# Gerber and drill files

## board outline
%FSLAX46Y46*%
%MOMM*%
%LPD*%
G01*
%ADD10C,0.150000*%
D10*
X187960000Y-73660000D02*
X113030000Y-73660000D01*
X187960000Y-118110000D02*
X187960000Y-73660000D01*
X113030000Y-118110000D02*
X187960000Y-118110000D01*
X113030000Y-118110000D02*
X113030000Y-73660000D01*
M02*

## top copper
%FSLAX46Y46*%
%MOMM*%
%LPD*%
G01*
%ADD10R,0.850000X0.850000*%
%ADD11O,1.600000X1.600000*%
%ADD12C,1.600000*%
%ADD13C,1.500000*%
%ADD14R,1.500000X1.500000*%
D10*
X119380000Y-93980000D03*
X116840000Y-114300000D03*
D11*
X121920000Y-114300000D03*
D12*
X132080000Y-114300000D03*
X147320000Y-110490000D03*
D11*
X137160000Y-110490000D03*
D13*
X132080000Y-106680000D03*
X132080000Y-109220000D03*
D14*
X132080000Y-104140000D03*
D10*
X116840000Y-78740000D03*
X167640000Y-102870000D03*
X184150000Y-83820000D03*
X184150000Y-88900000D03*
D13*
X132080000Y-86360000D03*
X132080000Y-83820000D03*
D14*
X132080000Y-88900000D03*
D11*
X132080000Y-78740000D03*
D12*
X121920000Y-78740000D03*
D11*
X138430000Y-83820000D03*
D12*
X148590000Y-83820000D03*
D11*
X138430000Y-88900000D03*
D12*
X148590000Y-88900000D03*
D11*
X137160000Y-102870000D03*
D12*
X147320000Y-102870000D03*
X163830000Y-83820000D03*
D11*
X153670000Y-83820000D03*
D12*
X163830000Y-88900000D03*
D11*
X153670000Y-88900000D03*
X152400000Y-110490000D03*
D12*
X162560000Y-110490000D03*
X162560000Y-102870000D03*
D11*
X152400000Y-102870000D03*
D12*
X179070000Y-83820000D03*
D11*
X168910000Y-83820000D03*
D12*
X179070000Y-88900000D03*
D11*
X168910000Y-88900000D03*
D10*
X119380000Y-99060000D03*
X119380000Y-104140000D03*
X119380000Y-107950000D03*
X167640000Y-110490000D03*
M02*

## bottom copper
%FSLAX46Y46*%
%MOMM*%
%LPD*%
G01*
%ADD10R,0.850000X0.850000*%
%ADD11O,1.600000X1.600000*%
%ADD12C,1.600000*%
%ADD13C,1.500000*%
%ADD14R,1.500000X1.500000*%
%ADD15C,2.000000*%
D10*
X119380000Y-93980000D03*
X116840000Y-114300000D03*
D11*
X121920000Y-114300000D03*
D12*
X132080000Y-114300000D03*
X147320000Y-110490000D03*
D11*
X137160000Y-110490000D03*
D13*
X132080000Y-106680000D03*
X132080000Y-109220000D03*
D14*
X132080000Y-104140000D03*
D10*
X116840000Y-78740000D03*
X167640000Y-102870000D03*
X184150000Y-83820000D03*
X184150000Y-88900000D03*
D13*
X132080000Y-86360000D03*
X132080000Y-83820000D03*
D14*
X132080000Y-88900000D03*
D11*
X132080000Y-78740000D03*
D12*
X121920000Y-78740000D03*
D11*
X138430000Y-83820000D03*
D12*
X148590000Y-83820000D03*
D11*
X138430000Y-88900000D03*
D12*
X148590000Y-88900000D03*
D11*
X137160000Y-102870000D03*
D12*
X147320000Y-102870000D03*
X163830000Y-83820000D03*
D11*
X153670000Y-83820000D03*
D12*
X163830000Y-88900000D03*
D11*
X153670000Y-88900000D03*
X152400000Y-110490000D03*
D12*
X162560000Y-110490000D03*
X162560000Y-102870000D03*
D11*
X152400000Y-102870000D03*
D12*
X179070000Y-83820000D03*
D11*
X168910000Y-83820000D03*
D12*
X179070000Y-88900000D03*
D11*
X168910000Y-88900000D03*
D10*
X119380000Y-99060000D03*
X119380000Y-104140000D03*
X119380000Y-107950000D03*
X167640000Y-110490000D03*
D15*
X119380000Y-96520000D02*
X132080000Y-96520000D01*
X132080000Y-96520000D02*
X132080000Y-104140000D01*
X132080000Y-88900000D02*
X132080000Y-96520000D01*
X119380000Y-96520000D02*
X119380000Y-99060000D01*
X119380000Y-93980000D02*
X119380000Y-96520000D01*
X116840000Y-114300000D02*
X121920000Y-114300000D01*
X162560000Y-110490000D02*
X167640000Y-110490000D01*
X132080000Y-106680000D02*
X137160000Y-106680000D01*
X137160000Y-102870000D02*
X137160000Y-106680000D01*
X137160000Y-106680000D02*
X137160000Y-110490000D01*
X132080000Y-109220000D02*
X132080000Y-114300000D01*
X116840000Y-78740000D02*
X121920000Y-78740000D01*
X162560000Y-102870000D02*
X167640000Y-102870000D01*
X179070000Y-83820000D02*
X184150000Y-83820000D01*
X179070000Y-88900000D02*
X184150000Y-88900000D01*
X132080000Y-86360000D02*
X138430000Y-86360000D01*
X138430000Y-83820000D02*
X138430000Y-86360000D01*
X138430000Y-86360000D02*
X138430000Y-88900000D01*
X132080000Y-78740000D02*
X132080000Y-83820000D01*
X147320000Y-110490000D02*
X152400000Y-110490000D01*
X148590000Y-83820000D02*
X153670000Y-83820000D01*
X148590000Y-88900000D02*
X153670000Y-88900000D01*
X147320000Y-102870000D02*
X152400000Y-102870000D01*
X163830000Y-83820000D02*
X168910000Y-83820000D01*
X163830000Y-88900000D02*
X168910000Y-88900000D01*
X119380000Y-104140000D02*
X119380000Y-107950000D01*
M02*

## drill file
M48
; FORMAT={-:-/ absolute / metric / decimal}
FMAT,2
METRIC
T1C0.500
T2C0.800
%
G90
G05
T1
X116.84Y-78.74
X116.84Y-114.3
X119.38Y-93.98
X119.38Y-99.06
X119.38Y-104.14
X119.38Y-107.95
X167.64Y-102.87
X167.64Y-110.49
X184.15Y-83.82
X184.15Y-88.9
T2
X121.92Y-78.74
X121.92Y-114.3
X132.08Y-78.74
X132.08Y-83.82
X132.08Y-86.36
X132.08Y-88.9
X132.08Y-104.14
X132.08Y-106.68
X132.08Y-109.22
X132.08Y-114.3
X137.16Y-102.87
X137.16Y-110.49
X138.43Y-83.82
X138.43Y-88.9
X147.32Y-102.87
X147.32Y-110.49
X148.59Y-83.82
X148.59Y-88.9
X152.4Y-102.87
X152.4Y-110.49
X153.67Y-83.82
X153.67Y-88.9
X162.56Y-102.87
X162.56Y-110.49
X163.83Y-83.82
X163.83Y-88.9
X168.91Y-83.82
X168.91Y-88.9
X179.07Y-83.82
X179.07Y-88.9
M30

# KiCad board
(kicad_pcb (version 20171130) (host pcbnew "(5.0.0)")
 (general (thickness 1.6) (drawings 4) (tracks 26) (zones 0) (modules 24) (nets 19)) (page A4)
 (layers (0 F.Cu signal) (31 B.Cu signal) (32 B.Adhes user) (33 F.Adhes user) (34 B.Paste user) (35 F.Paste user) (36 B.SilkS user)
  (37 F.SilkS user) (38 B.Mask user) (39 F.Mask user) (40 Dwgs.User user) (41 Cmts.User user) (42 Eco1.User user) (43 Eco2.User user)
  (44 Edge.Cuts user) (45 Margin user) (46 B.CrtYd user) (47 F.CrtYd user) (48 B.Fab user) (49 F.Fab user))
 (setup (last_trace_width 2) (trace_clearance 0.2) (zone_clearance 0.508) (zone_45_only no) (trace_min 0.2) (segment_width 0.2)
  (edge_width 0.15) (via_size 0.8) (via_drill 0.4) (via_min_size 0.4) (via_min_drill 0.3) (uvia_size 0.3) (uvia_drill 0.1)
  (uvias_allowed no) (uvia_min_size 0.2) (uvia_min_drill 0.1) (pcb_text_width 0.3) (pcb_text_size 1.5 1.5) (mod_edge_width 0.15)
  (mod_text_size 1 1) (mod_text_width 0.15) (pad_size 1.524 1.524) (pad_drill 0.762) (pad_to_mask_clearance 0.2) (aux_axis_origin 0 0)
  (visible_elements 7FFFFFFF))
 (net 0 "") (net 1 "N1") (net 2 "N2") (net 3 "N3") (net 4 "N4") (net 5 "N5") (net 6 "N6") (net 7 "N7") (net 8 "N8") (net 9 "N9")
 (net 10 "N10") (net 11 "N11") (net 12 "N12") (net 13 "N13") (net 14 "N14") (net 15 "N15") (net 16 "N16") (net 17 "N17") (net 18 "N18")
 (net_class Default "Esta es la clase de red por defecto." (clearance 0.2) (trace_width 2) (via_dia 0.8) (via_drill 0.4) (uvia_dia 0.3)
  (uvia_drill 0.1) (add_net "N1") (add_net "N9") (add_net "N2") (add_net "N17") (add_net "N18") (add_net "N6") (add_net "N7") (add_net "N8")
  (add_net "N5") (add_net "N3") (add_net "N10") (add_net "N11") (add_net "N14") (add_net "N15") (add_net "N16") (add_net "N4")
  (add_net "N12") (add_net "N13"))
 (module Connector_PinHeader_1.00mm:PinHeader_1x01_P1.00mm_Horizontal (layer F.Cu) (at 119.38 93.98 180)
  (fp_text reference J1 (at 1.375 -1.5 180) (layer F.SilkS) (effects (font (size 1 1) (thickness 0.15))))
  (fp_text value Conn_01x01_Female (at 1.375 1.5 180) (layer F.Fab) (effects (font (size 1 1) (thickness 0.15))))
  (pad 1 thru_hole rect (at 0 0 180) (size 0.85 0.85) (drill 0.5) (layers *.Cu *.Mask) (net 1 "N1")))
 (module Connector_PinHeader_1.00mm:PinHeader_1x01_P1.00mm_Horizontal (layer F.Cu) (at 116.84 114.3 180)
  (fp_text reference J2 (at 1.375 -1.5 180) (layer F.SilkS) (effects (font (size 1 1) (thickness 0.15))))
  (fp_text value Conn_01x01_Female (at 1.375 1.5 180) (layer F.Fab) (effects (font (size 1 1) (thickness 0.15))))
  (pad 1 thru_hole rect (at 0 0 180) (size 0.85 0.85) (drill 0.5) (layers *.Cu *.Mask) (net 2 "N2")))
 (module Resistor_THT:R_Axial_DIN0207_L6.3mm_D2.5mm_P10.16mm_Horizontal (layer F.Cu) (at 132.08 114.3 180)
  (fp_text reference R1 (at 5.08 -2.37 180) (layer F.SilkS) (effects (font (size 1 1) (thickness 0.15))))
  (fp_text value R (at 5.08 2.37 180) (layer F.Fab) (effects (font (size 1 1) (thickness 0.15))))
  (pad 2 thru_hole oval (at 10.16 0 180) (size 1.6 1.6) (drill 0.8) (layers *.Cu *.Mask) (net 2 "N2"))
  (pad 1 thru_hole circle (at 0 0 180) (size 1.6 1.6) (drill 0.8) (layers *.Cu *.Mask) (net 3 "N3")))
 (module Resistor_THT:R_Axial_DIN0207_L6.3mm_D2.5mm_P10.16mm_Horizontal (layer F.Cu) (at 147.32 110.49 180)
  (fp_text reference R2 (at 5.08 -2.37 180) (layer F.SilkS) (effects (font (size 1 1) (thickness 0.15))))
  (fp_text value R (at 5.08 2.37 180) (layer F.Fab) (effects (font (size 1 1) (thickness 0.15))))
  (pad 1 thru_hole circle (at 0 0 180) (size 1.6 1.6) (drill 0.8) (layers *.Cu *.Mask) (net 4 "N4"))
  (pad 2 thru_hole oval (at 10.16 0 180) (size 1.6 1.6) (drill 0.8) (layers *.Cu *.Mask) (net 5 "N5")))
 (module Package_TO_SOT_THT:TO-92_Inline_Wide (layer F.Cu) (at 132.08 104.14 270)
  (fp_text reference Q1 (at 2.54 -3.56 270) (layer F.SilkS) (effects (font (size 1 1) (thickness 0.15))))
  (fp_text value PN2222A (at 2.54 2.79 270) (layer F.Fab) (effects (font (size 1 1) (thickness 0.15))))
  (pad 2 thru_hole circle (at 2.54 0) (size 1.5 1.5) (drill 0.8) (layers *.Cu *.Mask) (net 5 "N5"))
  (pad 3 thru_hole circle (at 5.08 0) (size 1.5 1.5) (drill 0.8) (layers *.Cu *.Mask) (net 3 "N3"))
  (pad 1 thru_hole rect (at 0 0) (size 1.5 1.5) (drill 0.8) (layers *.Cu *.Mask) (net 1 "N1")))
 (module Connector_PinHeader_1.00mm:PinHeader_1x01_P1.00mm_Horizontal (layer F.Cu) (at 116.84 78.74 180)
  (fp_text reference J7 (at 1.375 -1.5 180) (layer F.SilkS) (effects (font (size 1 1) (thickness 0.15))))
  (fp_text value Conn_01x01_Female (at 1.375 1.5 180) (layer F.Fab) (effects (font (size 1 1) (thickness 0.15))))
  (pad 1 thru_hole rect (at 0 0 180) (size 0.85 0.85) (drill 0.5) (layers *.Cu *.Mask) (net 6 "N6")))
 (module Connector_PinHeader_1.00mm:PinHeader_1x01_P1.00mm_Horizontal (layer F.Cu) (at 167.64 102.87)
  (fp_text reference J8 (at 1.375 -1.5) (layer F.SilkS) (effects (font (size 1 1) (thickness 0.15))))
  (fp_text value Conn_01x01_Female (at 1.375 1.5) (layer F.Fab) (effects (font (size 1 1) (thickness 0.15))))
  (pad 1 thru_hole rect (at 0 0) (size 0.85 0.85) (drill 0.5) (layers *.Cu *.Mask) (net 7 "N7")))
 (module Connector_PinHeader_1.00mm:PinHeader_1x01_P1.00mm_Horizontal (layer F.Cu) (at 184.15 83.82)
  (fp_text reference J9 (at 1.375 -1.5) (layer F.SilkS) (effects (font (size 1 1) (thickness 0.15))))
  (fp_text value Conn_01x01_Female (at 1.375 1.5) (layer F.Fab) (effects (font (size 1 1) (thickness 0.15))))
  (pad 1 thru_hole rect (at 0 0) (size 0.85 0.85) (drill 0.5) (layers *.Cu *.Mask) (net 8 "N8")))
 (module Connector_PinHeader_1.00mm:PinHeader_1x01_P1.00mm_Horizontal (layer F.Cu) (at 184.15 88.9)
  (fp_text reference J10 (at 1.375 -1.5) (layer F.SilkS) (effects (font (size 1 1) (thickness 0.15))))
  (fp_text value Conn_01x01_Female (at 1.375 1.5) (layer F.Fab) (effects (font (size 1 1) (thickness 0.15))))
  (pad 1 thru_hole rect (at 0 0) (size 0.85 0.85) (drill 0.5) (layers *.Cu *.Mask) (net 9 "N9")))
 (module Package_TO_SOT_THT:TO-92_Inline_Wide (layer F.Cu) (at 132.08 88.9 90)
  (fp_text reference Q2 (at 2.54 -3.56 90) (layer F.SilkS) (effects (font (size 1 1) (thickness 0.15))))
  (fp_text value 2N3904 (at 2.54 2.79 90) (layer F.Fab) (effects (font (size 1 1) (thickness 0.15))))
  (pad 2 thru_hole circle (at 2.54 0 180) (size 1.5 1.5) (drill 0.8) (layers *.Cu *.Mask) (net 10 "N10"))
  (pad 3 thru_hole circle (at 5.08 0 180) (size 1.5 1.5) (drill 0.8) (layers *.Cu *.Mask) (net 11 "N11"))
  (pad 1 thru_hole rect (at 0 0 180) (size 1.5 1.5) (drill 0.8) (layers *.Cu *.Mask) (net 1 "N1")))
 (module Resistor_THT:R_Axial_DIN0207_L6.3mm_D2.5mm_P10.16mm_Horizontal (layer F.Cu) (at 121.92 78.74)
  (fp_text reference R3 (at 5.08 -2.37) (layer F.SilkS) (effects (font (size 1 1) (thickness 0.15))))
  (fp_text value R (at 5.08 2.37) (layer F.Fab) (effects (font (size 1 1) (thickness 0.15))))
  (pad 2 thru_hole oval (at 10.16 0) (size 1.6 1.6) (drill 0.8) (layers *.Cu *.Mask) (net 11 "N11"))
  (pad 1 thru_hole circle (at 0 0) (size 1.6 1.6) (drill 0.8) (layers *.Cu *.Mask) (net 6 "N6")))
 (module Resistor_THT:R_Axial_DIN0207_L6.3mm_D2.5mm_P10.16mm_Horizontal (layer F.Cu) (at 148.59 83.82 180)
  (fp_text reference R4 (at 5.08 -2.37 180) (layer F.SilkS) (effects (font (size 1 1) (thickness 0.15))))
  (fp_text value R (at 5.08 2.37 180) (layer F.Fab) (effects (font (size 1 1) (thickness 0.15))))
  (pad 2 thru_hole oval (at 10.16 0 180) (size 1.6 1.6) (drill 0.8) (layers *.Cu *.Mask) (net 10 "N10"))
  (pad 1 thru_hole circle (at 0 0 180) (size 1.6 1.6) (drill 0.8) (layers *.Cu *.Mask) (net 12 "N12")))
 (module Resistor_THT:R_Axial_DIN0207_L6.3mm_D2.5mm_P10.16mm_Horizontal (layer F.Cu) (at 148.59 88.9 180)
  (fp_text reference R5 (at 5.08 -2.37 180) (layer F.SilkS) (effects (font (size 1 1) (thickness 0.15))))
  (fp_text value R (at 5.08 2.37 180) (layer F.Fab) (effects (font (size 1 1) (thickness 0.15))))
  (pad 2 thru_hole oval (at 10.16 0 180) (size 1.6 1.6) (drill 0.8) (layers *.Cu *.Mask) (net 10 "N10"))
  (pad 1 thru_hole circle (at 0 0 180) (size 1.6 1.6) (drill 0.8) (layers *.Cu *.Mask) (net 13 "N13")))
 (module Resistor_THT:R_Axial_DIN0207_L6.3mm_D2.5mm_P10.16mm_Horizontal (layer F.Cu) (at 147.32 102.87 180)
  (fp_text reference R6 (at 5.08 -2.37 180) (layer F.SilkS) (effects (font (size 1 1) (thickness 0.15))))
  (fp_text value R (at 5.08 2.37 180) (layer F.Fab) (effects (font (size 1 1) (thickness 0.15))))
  (pad 2 thru_hole oval (at 10.16 0 180) (size 1.6 1.6) (drill 0.8) (layers *.Cu *.Mask) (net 5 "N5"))
  (pad 1 thru_hole circle (at 0 0 180) (size 1.6 1.6) (drill 0.8) (layers *.Cu *.Mask) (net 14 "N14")))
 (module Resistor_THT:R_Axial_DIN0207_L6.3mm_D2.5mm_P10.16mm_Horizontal (layer F.Cu) (at 163.83 83.82 180)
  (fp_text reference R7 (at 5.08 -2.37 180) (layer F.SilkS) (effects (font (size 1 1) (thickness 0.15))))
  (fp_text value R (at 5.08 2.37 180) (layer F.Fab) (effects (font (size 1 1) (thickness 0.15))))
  (pad 1 thru_hole circle (at 0 0 180) (size 1.6 1.6) (drill 0.8) (layers *.Cu *.Mask) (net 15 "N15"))
  (pad 2 thru_hole oval (at 10.16 0 180) (size 1.6 1.6) (drill 0.8) (layers *.Cu *.Mask) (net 12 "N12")))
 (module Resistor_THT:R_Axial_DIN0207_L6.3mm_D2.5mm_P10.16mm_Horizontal (layer F.Cu) (at 163.83 88.9 180)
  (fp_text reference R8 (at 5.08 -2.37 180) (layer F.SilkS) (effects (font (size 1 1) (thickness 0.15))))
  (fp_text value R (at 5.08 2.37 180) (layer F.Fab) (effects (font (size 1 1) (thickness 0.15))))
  (pad 1 thru_hole circle (at 0 0 180) (size 1.6 1.6) (drill 0.8) (layers *.Cu *.Mask) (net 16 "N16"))
  (pad 2 thru_hole oval (at 10.16 0 180) (size 1.6 1.6) (drill 0.8) (layers *.Cu *.Mask) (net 13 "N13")))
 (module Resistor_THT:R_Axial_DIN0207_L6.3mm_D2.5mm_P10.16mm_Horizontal (layer F.Cu) (at 162.56 110.49 180)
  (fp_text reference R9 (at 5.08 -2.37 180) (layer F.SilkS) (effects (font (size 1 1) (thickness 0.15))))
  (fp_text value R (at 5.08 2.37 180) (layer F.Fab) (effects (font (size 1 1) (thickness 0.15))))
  (pad 2 thru_hole oval (at 10.16 0 180) (size 1.6 1.6) (drill 0.8) (layers *.Cu *.Mask) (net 4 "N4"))
  (pad 1 thru_hole circle (at 0 0 180) (size 1.6 1.6) (drill 0.8) (layers *.Cu *.Mask) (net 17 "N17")))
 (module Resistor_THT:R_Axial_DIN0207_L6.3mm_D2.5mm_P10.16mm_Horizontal (layer F.Cu) (at 162.56 102.87 180)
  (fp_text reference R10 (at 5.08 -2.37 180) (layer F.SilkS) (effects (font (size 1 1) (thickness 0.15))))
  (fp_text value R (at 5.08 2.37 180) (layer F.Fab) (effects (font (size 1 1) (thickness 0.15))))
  (pad 1 thru_hole circle (at 0 0 180) (size 1.6 1.6) (drill 0.8) (layers *.Cu *.Mask) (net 7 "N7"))
  (pad 2 thru_hole oval (at 10.16 0 180) (size 1.6 1.6) (drill 0.8) (layers *.Cu *.Mask) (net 14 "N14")))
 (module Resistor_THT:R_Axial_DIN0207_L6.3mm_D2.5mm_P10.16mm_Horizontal (layer F.Cu) (at 179.07 83.82 180)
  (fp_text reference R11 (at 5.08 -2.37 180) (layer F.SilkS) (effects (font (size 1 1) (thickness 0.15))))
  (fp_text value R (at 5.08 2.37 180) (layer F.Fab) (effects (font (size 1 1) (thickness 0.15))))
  (pad 1 thru_hole circle (at 0 0 180) (size 1.6 1.6) (drill 0.8) (layers *.Cu *.Mask) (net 8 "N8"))
  (pad 2 thru_hole oval (at 10.16 0 180) (size 1.6 1.6) (drill 0.8) (layers *.Cu *.Mask) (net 15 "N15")))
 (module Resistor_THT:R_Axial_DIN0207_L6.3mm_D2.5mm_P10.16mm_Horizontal (layer F.Cu) (at 179.07 88.9 180)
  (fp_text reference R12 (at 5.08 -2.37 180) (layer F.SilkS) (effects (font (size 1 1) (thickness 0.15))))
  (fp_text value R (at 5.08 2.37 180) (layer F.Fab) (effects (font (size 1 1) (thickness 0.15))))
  (pad 1 thru_hole circle (at 0 0 180) (size 1.6 1.6) (drill 0.8) (layers *.Cu *.Mask) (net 9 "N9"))
  (pad 2 thru_hole oval (at 10.16 0 180) (size 1.6 1.6) (drill 0.8) (layers *.Cu *.Mask) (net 16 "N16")))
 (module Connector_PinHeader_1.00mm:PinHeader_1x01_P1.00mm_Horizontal (layer F.Cu) (at 119.38 99.06 180)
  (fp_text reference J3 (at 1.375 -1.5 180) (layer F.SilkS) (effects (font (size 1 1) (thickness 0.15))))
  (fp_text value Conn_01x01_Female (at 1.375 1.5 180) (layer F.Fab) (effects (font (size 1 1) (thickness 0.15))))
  (pad 1 thru_hole rect (at 0 0 180) (size 0.85 0.85) (drill 0.5) (layers *.Cu *.Mask) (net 1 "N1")))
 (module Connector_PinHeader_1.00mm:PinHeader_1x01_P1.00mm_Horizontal (layer F.Cu) (at 119.38 104.14 180)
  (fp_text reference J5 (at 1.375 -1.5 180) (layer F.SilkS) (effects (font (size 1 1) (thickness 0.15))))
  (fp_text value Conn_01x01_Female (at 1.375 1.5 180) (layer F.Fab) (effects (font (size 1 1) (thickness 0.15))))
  (pad 1 thru_hole rect (at 0 0 180) (size 0.85 0.85) (drill 0.5) (layers *.Cu *.Mask) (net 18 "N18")))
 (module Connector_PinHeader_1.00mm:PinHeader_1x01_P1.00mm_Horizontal (layer F.Cu) (at 119.38 107.95 180)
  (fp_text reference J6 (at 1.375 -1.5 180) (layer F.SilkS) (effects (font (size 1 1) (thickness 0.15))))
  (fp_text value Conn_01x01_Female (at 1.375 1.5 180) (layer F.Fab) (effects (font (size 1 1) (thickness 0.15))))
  (pad 1 thru_hole rect (at 0 0 180) (size 0.85 0.85) (drill 0.5) (layers *.Cu *.Mask) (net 18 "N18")))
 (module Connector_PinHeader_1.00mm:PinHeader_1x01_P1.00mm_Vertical (layer F.Cu) (at 167.64 110.49)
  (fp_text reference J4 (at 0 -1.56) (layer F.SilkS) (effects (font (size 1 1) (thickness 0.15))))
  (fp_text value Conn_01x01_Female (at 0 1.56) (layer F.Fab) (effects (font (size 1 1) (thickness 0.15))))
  (pad 1 thru_hole rect (at 0 0) (size 0.85 0.85) (drill 0.5) (layers *.Cu *.Mask) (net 17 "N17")))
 (gr_line (start 187.96 73.66) (end 113.03 73.66) (layer Edge.Cuts) (width 0.15))
 (gr_line (start 187.96 118.11) (end 187.96 73.66) (layer Edge.Cuts) (width 0.15))
 (gr_line (start 113.03 118.11) (end 187.96 118.11) (layer Edge.Cuts) (width 0.15))
 (gr_line (start 113.03 118.11) (end 113.03 73.66) (layer Edge.Cuts) (width 0.15))
 (segment (start 119.38 96.52) (end 132.08 96.52) (width 2) (layer B.Cu) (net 1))
 (segment (start 132.08 96.52) (end 132.08 104.14) (width 2) (layer B.Cu) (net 1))
 (segment (start 132.08 88.9) (end 132.08 96.52) (width 2) (layer B.Cu) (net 1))
 (segment (start 119.38 96.52) (end 119.38 99.06) (width 2) (layer B.Cu) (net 1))
 (segment (start 119.38 93.98) (end 119.38 96.52) (width 2) (layer B.Cu) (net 1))
 (segment (start 116.84 114.3) (end 121.92 114.3) (width 2) (layer B.Cu) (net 2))
 (segment (start 162.56 110.49) (end 167.64 110.49) (width 2) (layer B.Cu) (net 17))
 (segment (start 132.08 106.68) (end 137.16 106.68) (width 2) (layer B.Cu) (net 5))
 (segment (start 137.16 102.87) (end 137.16 106.68) (width 2) (layer B.Cu) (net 5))
 (segment (start 137.16 106.68) (end 137.16 110.49) (width 2) (layer B.Cu) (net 5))
 (segment (start 132.08 109.22) (end 132.08 114.3) (width 2) (layer B.Cu) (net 3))
 (segment (start 116.84 78.74) (end 121.92 78.74) (width 2) (layer B.Cu) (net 6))
 (segment (start 162.56 102.87) (end 167.64 102.87) (width 2) (layer B.Cu) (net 7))
 (segment (start 179.07 83.82) (end 184.15 83.82) (width 2) (layer B.Cu) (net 8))
 (segment (start 179.07 88.9) (end 184.15 88.9) (width 2) (layer B.Cu) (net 9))
 (segment (start 132.08 86.36) (end 138.43 86.36) (width 2) (layer B.Cu) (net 10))
 (segment (start 138.43 83.82) (end 138.43 86.36) (width 2) (layer B.Cu) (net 10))
 (segment (start 138.43 86.36) (end 138.43 88.9) (width 2) (layer B.Cu) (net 10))
 (segment (start 132.08 78.74) (end 132.08 83.82) (width 2) (layer B.Cu) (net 11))
 (segment (start 147.32 110.49) (end 152.4 110.49) (width 2) (layer B.Cu) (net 4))
 (segment (start 148.59 83.82) (end 153.67 83.82) (width 2) (layer B.Cu) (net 12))
 (segment (start 148.59 88.9) (end 153.67 88.9) (width 2) (layer B.Cu) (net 13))
 (segment (start 147.32 102.87) (end 152.4 102.87) (width 2) (layer B.Cu) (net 14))
 (segment (start 163.83 83.82) (end 168.91 83.82) (width 2) (layer B.Cu) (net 15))
 (segment (start 163.83 88.9) (end 168.91 88.9) (width 2) (layer B.Cu) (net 16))
 (segment (start 119.38 104.14) (end 119.38 107.95) (width 2) (layer B.Cu) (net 18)))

